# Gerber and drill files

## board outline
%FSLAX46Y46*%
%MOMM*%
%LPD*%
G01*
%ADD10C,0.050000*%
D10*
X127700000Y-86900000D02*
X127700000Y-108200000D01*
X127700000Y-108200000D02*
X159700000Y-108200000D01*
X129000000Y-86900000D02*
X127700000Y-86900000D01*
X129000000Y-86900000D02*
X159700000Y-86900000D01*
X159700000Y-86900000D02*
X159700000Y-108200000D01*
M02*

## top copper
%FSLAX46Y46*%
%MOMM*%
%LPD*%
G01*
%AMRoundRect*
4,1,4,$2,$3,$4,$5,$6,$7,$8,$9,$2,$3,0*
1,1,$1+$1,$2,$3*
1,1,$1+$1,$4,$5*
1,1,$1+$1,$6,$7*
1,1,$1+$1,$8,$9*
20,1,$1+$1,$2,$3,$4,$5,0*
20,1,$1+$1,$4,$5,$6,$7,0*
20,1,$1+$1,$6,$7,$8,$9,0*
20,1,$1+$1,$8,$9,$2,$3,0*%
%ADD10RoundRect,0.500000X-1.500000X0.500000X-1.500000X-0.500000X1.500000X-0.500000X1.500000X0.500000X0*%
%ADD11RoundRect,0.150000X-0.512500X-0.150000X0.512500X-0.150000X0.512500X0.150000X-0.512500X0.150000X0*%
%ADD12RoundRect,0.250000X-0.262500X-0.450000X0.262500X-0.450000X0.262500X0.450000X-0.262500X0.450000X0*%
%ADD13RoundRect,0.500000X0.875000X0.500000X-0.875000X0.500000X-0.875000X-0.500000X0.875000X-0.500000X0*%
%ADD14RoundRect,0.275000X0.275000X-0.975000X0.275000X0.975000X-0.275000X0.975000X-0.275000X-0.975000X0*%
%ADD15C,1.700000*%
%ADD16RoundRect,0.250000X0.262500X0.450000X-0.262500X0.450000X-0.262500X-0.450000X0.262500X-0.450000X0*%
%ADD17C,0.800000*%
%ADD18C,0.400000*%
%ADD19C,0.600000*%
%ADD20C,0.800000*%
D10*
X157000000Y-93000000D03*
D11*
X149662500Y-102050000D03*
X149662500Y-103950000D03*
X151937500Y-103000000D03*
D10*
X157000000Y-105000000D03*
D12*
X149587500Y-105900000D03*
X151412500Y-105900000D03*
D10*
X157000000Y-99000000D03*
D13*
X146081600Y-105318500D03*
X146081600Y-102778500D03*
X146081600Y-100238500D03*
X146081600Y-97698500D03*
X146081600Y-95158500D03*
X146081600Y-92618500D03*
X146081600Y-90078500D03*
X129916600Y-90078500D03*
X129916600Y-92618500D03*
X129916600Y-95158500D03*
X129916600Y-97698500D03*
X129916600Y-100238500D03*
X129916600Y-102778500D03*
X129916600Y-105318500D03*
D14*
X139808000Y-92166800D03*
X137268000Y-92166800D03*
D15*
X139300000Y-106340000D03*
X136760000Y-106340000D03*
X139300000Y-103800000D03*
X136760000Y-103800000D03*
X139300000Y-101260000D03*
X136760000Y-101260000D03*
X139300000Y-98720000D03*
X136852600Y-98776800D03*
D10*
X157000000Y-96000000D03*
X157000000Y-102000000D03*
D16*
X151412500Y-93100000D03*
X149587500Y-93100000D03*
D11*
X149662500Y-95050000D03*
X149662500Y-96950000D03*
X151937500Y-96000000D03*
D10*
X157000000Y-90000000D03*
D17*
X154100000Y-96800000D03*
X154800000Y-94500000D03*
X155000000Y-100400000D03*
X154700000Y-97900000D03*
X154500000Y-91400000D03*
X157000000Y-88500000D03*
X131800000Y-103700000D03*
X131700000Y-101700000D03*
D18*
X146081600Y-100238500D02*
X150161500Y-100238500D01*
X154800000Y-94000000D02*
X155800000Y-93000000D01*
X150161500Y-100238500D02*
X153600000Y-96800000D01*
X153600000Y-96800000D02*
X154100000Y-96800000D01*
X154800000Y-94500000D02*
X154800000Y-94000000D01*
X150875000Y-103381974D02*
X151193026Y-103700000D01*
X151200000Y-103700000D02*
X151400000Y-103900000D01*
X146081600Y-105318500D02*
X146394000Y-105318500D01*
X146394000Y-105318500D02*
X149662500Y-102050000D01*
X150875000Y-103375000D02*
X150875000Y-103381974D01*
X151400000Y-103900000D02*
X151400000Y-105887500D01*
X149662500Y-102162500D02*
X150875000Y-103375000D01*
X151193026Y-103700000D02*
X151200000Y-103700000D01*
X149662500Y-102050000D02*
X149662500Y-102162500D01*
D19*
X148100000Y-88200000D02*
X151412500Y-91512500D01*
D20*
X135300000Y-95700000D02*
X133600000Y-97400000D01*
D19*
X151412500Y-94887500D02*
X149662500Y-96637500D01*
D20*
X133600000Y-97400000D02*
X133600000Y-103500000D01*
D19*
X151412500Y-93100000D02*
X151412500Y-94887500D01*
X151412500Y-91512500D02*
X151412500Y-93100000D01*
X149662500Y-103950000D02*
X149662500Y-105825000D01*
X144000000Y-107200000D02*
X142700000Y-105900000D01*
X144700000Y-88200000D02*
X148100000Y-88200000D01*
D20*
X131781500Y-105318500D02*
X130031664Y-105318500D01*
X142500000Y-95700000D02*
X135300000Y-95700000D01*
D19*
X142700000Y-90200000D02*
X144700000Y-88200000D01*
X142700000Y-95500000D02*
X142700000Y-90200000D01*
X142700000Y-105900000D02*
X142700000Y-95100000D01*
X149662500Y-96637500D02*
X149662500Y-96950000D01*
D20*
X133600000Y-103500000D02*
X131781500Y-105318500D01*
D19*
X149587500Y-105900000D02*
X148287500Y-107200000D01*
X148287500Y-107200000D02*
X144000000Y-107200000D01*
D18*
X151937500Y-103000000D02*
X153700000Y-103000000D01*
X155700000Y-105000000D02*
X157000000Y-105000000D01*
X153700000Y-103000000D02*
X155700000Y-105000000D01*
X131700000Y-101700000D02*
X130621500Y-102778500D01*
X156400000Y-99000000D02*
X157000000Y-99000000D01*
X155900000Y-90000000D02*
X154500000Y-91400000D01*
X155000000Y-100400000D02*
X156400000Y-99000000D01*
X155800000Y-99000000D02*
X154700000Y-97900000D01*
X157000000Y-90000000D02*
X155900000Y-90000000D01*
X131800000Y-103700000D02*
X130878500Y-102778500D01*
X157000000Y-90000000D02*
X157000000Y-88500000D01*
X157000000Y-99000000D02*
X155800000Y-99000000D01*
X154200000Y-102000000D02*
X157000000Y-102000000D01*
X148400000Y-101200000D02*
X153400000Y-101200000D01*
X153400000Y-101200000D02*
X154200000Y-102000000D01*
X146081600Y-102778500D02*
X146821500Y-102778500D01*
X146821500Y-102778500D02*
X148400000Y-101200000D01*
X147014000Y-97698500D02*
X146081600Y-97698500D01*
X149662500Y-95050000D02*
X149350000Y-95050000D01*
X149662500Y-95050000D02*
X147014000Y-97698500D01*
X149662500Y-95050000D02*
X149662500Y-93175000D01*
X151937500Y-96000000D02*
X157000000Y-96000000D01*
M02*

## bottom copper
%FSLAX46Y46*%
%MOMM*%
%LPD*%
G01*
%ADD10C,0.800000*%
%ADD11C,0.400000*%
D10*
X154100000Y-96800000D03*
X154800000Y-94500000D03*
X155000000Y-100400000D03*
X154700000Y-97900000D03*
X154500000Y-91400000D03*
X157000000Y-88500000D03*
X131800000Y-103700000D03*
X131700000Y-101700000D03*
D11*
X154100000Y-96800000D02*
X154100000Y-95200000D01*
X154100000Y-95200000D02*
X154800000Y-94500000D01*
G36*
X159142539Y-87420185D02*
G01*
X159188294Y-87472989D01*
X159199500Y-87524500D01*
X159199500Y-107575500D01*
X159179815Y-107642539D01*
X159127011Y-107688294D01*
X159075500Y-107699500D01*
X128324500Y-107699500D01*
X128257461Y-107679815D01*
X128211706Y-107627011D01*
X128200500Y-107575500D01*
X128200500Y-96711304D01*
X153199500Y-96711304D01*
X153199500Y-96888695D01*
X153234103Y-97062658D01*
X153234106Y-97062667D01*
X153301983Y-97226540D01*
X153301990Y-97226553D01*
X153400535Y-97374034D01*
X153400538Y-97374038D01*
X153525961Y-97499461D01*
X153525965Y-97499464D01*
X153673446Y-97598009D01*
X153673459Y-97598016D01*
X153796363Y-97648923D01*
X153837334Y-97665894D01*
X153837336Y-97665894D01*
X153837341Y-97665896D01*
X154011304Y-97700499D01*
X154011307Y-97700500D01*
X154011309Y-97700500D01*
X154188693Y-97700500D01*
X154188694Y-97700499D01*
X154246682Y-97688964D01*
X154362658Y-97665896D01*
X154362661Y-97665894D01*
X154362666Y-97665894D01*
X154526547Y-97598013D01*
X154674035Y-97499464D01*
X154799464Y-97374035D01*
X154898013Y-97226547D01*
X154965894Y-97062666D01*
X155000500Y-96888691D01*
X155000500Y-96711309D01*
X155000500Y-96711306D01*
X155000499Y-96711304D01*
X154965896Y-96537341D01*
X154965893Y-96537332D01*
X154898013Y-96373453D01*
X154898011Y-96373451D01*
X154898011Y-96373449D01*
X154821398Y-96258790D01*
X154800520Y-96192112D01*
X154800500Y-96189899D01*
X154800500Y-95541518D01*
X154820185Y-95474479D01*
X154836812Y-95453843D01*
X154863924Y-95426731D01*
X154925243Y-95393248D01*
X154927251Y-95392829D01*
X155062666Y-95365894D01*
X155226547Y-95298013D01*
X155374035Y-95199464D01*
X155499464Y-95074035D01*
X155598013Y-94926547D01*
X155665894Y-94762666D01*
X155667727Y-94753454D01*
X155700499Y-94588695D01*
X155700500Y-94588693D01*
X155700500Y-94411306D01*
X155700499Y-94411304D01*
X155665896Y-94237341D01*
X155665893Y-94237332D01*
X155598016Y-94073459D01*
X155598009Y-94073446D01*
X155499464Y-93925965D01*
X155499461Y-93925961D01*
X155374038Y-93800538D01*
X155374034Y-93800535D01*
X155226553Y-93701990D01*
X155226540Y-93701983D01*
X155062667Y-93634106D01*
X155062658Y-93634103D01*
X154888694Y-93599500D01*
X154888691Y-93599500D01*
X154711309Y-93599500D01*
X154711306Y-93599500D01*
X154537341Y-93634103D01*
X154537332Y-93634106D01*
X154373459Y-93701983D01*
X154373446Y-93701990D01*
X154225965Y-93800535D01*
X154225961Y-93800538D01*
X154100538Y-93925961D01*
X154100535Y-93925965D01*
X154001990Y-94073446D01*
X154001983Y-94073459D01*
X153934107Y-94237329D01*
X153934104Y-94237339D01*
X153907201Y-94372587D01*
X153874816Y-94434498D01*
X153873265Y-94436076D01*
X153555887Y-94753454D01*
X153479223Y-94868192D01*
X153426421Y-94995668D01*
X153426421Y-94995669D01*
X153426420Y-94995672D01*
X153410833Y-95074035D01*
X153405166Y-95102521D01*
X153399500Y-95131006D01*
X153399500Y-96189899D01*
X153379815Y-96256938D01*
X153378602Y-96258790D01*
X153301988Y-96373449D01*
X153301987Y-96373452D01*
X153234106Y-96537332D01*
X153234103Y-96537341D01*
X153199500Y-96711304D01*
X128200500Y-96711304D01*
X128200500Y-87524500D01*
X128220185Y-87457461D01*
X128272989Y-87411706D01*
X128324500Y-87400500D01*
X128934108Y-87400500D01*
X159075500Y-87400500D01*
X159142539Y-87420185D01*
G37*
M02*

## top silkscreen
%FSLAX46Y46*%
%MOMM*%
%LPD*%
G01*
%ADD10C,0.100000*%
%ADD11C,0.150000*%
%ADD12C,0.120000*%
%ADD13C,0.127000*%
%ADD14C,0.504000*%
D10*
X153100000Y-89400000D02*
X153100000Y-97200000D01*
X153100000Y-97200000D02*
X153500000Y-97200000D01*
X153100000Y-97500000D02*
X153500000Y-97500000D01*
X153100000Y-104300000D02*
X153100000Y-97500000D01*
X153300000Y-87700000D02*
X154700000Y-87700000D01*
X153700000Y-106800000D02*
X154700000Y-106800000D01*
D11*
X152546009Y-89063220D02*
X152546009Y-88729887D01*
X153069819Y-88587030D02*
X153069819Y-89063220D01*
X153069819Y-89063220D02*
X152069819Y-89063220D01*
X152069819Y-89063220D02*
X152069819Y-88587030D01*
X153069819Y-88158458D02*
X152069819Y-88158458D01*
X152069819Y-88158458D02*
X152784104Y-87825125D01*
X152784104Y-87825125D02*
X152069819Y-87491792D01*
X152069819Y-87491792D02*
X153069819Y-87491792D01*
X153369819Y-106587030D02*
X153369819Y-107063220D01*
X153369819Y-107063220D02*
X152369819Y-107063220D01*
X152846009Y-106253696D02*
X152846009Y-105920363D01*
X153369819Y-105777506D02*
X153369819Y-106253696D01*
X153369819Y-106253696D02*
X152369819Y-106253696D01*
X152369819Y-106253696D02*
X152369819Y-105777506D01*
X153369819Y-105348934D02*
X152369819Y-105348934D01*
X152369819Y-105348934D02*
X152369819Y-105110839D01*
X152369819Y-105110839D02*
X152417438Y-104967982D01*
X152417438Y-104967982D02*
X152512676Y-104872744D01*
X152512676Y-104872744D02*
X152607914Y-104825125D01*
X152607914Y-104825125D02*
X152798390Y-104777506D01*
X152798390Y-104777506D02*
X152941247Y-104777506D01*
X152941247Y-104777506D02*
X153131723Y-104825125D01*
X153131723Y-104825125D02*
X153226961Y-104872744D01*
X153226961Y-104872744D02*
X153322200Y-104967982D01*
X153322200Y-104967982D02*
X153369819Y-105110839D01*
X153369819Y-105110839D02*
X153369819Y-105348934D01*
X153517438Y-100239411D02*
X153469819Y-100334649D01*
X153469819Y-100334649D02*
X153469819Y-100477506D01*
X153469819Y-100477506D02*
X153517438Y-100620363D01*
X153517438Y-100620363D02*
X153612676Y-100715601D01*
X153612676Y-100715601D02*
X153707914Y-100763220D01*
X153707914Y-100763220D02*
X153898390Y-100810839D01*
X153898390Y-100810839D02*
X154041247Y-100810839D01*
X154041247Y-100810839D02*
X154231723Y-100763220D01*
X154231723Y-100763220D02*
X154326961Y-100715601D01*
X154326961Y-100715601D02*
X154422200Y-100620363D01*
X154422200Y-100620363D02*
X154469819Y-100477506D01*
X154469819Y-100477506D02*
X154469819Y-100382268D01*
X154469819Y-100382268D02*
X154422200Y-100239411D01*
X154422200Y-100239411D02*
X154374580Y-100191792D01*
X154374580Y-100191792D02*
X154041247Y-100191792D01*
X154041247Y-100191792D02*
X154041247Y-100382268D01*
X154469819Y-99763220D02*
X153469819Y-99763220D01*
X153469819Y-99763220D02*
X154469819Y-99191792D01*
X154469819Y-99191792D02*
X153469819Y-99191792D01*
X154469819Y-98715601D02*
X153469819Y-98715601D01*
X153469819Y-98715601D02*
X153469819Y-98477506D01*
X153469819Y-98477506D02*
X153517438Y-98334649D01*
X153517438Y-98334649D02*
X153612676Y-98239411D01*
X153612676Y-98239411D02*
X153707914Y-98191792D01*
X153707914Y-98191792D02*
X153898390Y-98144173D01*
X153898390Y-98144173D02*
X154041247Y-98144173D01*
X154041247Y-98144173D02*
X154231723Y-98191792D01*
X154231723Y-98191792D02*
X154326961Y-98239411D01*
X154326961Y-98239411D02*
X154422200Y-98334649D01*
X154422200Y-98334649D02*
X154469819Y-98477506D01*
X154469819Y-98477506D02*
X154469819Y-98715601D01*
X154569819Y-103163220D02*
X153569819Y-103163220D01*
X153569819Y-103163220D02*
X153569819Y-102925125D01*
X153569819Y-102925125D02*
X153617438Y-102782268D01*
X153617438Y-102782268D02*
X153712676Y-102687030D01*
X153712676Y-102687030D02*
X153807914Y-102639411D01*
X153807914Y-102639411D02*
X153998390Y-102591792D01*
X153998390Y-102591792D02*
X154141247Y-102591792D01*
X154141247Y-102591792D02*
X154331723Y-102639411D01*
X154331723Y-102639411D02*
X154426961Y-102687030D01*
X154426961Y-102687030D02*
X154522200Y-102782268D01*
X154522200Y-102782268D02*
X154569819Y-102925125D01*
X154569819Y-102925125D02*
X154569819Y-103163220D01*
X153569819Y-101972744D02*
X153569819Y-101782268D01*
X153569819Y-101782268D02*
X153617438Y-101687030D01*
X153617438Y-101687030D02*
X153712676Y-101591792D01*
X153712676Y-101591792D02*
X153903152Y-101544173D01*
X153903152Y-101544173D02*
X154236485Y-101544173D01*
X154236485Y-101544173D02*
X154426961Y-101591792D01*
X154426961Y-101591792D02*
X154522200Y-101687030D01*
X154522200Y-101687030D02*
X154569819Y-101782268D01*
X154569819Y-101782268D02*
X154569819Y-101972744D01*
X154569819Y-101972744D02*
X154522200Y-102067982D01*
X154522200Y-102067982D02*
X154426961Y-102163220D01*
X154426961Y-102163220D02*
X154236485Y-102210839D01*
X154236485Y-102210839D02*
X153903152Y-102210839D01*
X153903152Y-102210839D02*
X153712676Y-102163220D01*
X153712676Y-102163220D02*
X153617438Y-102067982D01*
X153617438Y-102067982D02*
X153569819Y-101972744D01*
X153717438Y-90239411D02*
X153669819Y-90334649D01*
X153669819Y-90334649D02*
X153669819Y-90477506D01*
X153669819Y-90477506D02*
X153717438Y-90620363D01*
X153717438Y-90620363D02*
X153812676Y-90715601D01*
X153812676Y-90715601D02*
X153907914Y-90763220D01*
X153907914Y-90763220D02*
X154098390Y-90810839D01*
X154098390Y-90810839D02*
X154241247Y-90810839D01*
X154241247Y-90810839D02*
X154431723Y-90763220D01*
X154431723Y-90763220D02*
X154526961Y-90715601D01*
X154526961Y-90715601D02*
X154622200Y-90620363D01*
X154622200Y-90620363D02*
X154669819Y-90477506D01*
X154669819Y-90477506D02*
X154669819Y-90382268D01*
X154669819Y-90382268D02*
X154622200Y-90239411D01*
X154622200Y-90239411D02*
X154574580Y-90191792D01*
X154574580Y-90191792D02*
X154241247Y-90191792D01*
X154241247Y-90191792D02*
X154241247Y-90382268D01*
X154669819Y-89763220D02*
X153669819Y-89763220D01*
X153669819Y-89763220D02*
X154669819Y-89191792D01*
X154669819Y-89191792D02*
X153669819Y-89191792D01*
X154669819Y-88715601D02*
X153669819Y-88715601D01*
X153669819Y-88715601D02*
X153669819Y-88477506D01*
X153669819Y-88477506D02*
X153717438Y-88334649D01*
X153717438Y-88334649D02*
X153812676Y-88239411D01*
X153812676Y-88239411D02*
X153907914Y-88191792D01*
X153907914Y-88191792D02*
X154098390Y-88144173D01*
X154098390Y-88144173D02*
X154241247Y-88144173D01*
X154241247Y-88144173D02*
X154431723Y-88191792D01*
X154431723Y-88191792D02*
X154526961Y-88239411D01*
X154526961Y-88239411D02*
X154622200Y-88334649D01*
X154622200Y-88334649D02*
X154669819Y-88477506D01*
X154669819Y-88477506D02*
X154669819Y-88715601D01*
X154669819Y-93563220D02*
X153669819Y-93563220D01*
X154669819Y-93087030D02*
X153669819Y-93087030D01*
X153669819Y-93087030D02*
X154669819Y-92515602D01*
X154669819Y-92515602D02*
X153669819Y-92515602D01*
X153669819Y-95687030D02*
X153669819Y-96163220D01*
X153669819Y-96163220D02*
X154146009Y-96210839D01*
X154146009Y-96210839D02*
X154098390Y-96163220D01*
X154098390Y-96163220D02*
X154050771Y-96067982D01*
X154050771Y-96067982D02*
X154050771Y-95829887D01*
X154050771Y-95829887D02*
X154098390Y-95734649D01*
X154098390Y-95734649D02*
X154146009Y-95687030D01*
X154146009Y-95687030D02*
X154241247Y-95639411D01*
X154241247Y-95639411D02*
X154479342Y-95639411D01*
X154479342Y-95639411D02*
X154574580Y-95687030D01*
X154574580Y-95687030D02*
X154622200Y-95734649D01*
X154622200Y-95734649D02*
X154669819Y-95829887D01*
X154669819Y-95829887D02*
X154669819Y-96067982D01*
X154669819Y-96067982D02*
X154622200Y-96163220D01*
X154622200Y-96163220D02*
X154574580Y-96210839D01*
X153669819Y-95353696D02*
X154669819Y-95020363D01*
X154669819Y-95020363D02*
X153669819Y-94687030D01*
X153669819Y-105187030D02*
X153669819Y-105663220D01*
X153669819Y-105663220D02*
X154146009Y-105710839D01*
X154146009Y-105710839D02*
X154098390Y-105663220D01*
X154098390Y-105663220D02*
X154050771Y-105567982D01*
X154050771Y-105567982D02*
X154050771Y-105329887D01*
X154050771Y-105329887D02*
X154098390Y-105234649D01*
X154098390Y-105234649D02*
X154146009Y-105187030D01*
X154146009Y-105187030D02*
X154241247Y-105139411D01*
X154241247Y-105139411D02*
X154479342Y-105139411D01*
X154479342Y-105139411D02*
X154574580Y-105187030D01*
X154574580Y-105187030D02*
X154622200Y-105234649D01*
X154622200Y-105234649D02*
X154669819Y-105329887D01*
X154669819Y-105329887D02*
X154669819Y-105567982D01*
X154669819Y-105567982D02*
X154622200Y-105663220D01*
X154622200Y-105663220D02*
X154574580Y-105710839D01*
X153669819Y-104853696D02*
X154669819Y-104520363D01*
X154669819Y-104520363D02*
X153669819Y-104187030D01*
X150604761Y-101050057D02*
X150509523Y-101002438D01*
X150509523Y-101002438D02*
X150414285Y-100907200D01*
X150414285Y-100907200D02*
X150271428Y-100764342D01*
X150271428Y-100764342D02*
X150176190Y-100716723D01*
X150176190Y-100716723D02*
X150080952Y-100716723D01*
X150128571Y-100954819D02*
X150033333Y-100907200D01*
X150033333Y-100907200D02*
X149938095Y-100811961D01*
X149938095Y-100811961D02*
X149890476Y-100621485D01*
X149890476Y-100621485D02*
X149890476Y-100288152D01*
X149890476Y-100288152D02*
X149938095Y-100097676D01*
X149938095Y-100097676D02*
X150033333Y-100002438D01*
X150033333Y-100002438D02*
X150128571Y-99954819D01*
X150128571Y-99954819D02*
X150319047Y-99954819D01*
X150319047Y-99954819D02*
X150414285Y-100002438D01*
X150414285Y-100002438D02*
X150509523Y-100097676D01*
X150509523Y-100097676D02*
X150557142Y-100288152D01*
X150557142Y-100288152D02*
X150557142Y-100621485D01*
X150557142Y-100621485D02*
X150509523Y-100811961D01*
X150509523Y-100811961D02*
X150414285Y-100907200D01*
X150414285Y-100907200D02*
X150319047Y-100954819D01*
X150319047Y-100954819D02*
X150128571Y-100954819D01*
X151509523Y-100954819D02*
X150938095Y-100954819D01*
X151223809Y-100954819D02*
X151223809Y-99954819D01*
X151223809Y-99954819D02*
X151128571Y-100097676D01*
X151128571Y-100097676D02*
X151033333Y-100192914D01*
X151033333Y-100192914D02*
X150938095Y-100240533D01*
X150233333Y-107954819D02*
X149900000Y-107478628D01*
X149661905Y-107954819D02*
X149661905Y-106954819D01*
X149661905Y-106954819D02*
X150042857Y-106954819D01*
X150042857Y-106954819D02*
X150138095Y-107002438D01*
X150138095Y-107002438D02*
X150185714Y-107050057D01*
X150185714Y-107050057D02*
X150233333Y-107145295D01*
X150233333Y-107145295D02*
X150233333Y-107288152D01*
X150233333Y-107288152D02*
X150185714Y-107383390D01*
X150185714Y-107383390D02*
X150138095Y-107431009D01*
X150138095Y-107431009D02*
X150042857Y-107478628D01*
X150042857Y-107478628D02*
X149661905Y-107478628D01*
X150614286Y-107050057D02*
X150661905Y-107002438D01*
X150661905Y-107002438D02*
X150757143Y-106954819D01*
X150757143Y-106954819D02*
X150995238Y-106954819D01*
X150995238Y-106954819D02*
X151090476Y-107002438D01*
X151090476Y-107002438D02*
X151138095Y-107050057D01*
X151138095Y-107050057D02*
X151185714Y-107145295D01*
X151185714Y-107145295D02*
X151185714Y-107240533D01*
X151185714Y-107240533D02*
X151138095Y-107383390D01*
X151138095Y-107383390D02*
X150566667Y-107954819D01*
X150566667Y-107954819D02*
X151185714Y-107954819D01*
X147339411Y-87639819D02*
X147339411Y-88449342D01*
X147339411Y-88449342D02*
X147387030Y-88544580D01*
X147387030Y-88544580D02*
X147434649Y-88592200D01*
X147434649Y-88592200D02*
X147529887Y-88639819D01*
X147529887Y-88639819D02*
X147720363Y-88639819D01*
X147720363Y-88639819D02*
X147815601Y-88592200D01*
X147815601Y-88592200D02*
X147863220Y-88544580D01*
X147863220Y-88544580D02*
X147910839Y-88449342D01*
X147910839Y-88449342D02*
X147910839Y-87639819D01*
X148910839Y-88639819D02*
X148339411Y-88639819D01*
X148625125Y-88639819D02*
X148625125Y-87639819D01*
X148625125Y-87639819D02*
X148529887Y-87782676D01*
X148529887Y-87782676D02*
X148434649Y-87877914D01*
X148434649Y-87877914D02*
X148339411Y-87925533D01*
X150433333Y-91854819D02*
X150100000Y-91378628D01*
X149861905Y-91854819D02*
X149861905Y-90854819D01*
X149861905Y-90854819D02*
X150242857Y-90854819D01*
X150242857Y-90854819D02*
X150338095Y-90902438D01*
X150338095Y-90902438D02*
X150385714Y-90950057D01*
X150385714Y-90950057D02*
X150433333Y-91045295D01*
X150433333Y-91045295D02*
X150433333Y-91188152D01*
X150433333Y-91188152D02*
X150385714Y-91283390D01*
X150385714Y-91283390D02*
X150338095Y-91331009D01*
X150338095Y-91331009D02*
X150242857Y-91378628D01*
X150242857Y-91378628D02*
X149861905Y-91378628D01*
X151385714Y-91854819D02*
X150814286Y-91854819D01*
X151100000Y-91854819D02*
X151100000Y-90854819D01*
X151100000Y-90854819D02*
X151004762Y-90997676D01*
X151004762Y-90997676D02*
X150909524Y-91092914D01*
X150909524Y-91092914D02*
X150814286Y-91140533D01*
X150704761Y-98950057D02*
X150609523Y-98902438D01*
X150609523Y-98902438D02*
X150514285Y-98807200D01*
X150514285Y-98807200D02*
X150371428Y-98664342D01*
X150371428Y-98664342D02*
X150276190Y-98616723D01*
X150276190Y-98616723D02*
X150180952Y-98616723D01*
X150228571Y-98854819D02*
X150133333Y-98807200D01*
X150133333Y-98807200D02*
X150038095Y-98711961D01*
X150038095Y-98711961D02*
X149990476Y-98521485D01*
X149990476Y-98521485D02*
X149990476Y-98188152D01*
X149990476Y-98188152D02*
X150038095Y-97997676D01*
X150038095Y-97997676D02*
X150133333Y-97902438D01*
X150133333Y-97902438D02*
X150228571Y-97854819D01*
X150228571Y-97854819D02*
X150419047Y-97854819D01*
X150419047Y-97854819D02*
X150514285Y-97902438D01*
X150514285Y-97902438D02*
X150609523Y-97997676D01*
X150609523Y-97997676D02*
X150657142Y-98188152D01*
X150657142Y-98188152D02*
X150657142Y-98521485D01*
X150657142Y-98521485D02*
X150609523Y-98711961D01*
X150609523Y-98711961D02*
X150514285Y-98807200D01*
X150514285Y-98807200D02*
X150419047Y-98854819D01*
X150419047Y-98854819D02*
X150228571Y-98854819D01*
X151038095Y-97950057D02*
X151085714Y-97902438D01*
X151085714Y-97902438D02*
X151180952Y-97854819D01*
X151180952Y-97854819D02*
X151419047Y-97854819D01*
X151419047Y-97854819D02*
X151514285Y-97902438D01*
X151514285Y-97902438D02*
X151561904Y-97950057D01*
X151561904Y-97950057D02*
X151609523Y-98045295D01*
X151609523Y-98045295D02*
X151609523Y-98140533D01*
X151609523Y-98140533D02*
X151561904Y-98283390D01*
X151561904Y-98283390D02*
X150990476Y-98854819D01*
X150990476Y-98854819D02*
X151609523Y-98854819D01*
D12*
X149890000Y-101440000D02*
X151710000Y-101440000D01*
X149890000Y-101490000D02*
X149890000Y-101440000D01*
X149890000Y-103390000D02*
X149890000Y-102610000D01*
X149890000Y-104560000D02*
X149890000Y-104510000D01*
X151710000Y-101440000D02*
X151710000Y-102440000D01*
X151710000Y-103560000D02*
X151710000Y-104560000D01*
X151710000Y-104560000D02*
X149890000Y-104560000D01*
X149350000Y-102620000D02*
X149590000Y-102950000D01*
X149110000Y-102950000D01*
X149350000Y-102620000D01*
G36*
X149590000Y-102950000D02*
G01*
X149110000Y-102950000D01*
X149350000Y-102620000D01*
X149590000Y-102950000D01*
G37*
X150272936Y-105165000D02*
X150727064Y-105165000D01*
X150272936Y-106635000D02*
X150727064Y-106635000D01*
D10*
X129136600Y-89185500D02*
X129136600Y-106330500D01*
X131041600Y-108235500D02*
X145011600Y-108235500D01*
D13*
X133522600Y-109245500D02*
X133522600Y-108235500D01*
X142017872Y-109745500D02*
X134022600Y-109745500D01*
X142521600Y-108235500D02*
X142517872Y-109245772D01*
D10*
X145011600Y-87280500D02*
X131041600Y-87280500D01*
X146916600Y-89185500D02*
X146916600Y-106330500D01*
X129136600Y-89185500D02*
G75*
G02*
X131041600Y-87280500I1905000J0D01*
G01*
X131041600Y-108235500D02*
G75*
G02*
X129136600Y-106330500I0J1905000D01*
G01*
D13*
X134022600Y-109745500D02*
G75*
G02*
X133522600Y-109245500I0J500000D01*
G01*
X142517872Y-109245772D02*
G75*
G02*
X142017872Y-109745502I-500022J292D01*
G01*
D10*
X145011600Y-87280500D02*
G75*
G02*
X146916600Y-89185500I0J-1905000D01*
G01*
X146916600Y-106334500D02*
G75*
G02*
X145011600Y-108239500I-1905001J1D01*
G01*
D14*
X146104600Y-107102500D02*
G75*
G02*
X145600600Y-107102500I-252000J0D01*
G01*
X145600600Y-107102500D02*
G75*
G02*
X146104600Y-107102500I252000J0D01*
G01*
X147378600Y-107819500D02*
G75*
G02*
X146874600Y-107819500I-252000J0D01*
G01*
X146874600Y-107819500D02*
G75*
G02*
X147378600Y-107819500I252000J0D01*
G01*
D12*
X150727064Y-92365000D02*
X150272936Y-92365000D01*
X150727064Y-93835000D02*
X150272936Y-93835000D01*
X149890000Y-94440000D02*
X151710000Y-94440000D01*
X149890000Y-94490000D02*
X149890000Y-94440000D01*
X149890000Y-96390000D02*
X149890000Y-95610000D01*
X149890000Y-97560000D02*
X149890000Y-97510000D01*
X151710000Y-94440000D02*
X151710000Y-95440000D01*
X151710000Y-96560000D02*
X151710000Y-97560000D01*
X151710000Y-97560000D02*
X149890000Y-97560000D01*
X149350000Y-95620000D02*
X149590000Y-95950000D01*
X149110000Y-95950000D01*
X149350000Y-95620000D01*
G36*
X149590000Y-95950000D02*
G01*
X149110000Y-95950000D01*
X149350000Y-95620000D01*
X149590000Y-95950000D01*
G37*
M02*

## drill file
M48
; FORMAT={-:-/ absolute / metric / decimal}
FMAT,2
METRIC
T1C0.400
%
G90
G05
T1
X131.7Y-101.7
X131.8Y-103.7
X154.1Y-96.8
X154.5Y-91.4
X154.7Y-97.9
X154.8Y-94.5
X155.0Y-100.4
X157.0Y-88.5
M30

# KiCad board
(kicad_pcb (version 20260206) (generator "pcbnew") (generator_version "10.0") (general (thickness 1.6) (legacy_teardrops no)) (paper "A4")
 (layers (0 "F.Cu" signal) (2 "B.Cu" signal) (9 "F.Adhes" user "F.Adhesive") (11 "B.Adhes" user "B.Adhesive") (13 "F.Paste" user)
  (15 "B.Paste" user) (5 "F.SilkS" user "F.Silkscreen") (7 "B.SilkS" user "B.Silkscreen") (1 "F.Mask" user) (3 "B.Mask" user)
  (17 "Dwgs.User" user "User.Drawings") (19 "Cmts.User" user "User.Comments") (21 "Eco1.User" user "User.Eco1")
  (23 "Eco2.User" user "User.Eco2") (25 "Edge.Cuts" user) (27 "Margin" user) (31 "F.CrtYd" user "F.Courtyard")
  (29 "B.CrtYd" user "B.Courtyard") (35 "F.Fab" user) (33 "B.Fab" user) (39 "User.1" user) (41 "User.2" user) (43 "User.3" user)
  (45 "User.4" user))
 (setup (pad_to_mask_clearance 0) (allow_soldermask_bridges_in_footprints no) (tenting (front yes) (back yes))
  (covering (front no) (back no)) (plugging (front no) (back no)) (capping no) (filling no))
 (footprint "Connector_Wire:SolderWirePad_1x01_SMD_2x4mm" (layer "F.Cu") (at 157 93 -90)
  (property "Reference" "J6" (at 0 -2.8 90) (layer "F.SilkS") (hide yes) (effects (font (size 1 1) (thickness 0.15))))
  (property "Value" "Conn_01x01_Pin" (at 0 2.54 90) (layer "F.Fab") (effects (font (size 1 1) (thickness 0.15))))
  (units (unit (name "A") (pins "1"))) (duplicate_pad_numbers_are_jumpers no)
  (pad "1" smd roundrect (at 0 0 270) (size 2 4) (layers "F.Cu" "F.Mask") (roundrect_rratio 0.25) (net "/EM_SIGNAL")))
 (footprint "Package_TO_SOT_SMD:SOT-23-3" (layer "F.Cu") (at 150.8 103)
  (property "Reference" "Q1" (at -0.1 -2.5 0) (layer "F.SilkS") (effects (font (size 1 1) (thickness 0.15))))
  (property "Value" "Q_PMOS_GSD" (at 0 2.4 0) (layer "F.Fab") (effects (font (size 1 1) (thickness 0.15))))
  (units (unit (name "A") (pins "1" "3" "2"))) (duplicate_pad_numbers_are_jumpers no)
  (fp_line (start -0.91 -1.56) (end 0.91 -1.56) (stroke (width 0.12) (type solid)) (layer "F.SilkS"))
  (fp_line (start -0.91 -1.51) (end -0.91 -1.56) (stroke (width 0.12) (type solid)) (layer "F.SilkS"))
  (fp_line (start -0.91 0.39) (end -0.91 -0.39) (stroke (width 0.12) (type solid)) (layer "F.SilkS"))
  (fp_line (start -0.91 1.56) (end -0.91 1.51) (stroke (width 0.12) (type solid)) (layer "F.SilkS"))
  (fp_line (start 0.91 -1.56) (end 0.91 -0.56) (stroke (width 0.12) (type solid)) (layer "F.SilkS"))
  (fp_line (start 0.91 0.56) (end 0.91 1.56) (stroke (width 0.12) (type solid)) (layer "F.SilkS"))
  (fp_line (start 0.91 1.56) (end -0.91 1.56) (stroke (width 0.12) (type solid)) (layer "F.SilkS"))
  (fp_poly (pts (xy -1.45 -0.38) (xy -1.21 -0.05) (xy -1.69 -0.05)) (stroke (width 0.12) (type solid)) (fill yes) (layer "F.SilkS"))
  (pad "1" smd roundrect (at -1.1375 -0.95) (size 1.325 0.6) (layers "F.Cu" "F.Mask" "F.Paste") (roundrect_rratio 0.25) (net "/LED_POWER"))
  (pad "2" smd roundrect (at -1.1375 0.95) (size 1.325 0.6) (layers "F.Cu" "F.Mask" "F.Paste") (roundrect_rratio 0.25) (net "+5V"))
  (pad "3" smd roundrect (at 1.1375 0) (size 1.325 0.6) (layers "F.Cu" "F.Mask" "F.Paste") (roundrect_rratio 0.25) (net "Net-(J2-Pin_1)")))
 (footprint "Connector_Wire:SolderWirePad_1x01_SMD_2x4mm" (layer "F.Cu") (at 157 105 -90)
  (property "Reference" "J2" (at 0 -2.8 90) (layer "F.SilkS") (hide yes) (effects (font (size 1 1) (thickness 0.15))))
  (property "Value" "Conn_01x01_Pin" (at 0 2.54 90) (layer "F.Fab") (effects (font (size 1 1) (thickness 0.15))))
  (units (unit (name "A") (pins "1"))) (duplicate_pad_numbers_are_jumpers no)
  (pad "1" smd roundrect (at 0 0 270) (size 2 4) (layers "F.Cu" "F.Mask") (roundrect_rratio 0.25) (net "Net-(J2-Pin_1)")))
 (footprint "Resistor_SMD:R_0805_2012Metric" (layer "F.Cu") (at 150.5 105.9)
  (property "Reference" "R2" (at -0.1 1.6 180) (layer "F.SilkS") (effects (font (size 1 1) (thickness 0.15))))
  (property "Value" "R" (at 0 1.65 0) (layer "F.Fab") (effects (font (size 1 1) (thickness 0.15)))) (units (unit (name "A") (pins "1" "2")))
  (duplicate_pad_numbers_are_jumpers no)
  (fp_line (start -0.227064 -0.735) (end 0.227064 -0.735) (stroke (width 0.12) (type solid)) (layer "F.SilkS"))
  (fp_line (start -0.227064 0.735) (end 0.227064 0.735) (stroke (width 0.12) (type solid)) (layer "F.SilkS"))
  (pad "1" smd roundrect (at -0.9125 0) (size 1.025 1.4) (layers "F.Cu" "F.Mask" "F.Paste") (roundrect_rratio 0.243902) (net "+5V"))
  (pad "2" smd roundrect (at 0.9125 0) (size 1.025 1.4) (layers "F.Cu" "F.Mask" "F.Paste") (roundrect_rratio 0.243902) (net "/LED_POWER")))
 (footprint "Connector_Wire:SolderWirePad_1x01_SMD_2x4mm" (layer "F.Cu") (at 157 99 -90)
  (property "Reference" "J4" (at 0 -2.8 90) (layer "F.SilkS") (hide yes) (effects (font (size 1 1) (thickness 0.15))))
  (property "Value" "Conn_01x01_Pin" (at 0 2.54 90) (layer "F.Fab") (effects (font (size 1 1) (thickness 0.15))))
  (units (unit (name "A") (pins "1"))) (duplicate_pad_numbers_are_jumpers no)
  (pad "1" smd roundrect (at 0 0 270) (size 2 4) (layers "F.Cu" "F.Mask") (roundrect_rratio 0.25) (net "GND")))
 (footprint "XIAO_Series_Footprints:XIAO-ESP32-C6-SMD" (layer "F.Cu") (at 146.9166 87.1985 180)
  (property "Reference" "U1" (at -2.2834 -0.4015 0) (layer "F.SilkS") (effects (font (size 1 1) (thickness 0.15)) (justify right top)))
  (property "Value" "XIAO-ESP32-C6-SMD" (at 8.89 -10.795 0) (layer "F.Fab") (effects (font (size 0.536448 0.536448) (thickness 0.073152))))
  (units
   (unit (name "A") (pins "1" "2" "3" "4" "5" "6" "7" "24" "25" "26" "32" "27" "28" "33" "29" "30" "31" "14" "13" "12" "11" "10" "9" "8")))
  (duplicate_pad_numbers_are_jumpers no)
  (fp_line (start 17.78 -1.987) (end 17.78 -19.132) (stroke (width 0.1) (type solid)) (layer "F.SilkS"))
  (fp_line (start 15.875 -21.037) (end 1.905 -21.037) (stroke (width 0.1) (type solid)) (layer "F.SilkS"))
  (fp_line (start 13.394 -22.047) (end 13.394 -21.037) (stroke (width 0.127) (type solid)) (layer "F.SilkS"))
  (fp_line (start 4.898728 -22.547) (end 12.894 -22.547) (stroke (width 0.127) (type solid)) (layer "F.SilkS"))
  (fp_line (start 4.395 -21.037) (end 4.398728 -22.047272) (stroke (width 0.127) (type solid)) (layer "F.SilkS"))
  (fp_line (start 1.905 -0.082) (end 15.875 -0.082) (stroke (width 0.1) (type solid)) (layer "F.SilkS"))
  (fp_line (start 0 -1.987) (end 0 -19.132) (stroke (width 0.1) (type solid)) (layer "F.SilkS"))
  (fp_arc (start 17.78 -1.987) (mid 17.222038 -0.639962) (end 15.875 -0.082) (stroke (width 0.1) (type solid)) (layer "F.SilkS"))
  (fp_arc (start 15.875 -21.037) (mid 17.222038 -20.479038) (end 17.78 -19.132) (stroke (width 0.1) (type solid)) (layer "F.SilkS"))
  (fp_arc (start 12.894 -22.547) (mid 13.247553 -22.400553) (end 13.394 -22.047) (stroke (width 0.127) (type default)) (layer "F.SilkS"))
  (fp_arc (start 4.398728 -22.047272) (mid 4.545276 -22.400644) (end 4.898728 -22.547) (stroke (width 0.127) (type default))
   (layer "F.SilkS"))
  (fp_arc (start 1.905 -0.082) (mid 0.557962 -0.639962) (end 0 -1.987) (stroke (width 0.1) (type solid)) (layer "F.SilkS"))
  (fp_arc (start 0 -19.136) (mid 0.557962 -20.483038) (end 1.905 -21.041) (stroke (width 0.1) (type solid)) (layer "F.SilkS"))
  (fp_circle (center 1.064 -19.904) (end 1.064 -20.158) (stroke (width 0.5) (type solid)) (fill yes) (layer "F.SilkS"))
  (fp_circle (center -0.21 -20.621) (end -0.21 -20.875) (stroke (width 0.5) (type solid)) (fill yes) (layer "F.SilkS"))
  (pad "1" smd roundrect (at 0.835 -18.12 180) (size 2.75 2) (layers "F.Cu" "F.Mask" "F.Paste") (roundrect_rratio 0.25) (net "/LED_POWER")
   (solder_mask_margin 0.0508) (thermal_bridge_angle 45))
  (pad "2" smd roundrect (at 0.835 -15.58 180) (size 2.75 2) (layers "F.Cu" "F.Mask" "F.Paste") (roundrect_rratio 0.25) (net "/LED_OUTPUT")
   (solder_mask_margin 0.0508) (thermal_bridge_angle 45))
  (pad "3" smd roundrect (at 0.835 -13.04 180) (size 2.75 2) (layers "F.Cu" "F.Mask" "F.Paste") (roundrect_rratio 0.25) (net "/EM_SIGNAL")
   (solder_mask_margin 0.0508) (thermal_bridge_angle 45))
  (pad "4" smd roundrect (at 0.835 -10.5 180) (size 2.75 2) (layers "F.Cu" "F.Mask" "F.Paste") (roundrect_rratio 0.25) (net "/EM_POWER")
   (solder_mask_margin 0.0508) (thermal_bridge_angle 45))
  (pad "5" smd roundrect (at 0.835 -7.96 180) (size 2.75 2) (layers "F.Cu" "F.Mask" "F.Paste") (roundrect_rratio 0.25)
   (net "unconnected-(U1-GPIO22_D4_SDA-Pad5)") (solder_mask_margin 0.0508) (thermal_bridge_angle 45))
  (pad "6" smd roundrect (at 0.835 -5.42 180) (size 2.75 2) (layers "F.Cu" "F.Mask" "F.Paste") (roundrect_rratio 0.25)
   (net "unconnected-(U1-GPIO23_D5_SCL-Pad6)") (solder_mask_margin 0.0508) (thermal_bridge_angle 45))
  (pad "7" smd roundrect (at 0.835 -2.88 180) (size 2.75 2) (layers "F.Cu" "F.Mask" "F.Paste") (roundrect_rratio 0.25)
   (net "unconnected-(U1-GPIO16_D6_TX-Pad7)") (solder_mask_margin 0.0508) (thermal_bridge_angle 45))
  (pad "8" smd roundrect (at 17 -2.88 180) (size 2.75 2) (layers "F.Cu" "F.Mask" "F.Paste") (roundrect_rratio 0.25)
   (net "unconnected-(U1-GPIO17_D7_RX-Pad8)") (solder_mask_margin 0.0508) (thermal_bridge_angle 45))
  (pad "9" smd roundrect (at 17 -5.42 180) (size 2.75 2) (layers "F.Cu" "F.Mask" "F.Paste") (roundrect_rratio 0.25)
   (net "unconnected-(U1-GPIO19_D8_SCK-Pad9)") (solder_mask_margin 0.0508) (thermal_bridge_angle 45))
  (pad "10" smd roundrect (at 17 -7.96 180) (size 2.75 2) (layers "F.Cu" "F.Mask" "F.Paste") (roundrect_rratio 0.25)
   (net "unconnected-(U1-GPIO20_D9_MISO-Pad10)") (solder_mask_margin 0.0508) (thermal_bridge_angle 45))
  (pad "11" smd roundrect (at 17 -10.5 180) (size 2.75 2) (layers "F.Cu" "F.Mask" "F.Paste") (roundrect_rratio 0.25)
   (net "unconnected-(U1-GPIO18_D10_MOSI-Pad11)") (solder_mask_margin 0.0508) (thermal_bridge_angle 45))
  (pad "12" smd roundrect (at 17 -13.04 180) (size 2.75 2) (layers "F.Cu" "F.Mask" "F.Paste") (roundrect_rratio 0.25)
   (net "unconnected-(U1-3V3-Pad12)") (solder_mask_margin 0.0508) (thermal_bridge_angle 45))
  (pad "13" smd roundrect (at 17 -15.58 180) (size 2.75 2) (layers "F.Cu" "F.Mask" "F.Paste") (roundrect_rratio 0.25) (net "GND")
   (solder_mask_margin 0.0508) (thermal_bridge_angle 45))
  (pad "14" smd roundrect (at 17 -18.12 180) (size 2.75 2) (layers "F.Cu" "F.Mask" "F.Paste") (roundrect_rratio 0.25) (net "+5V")
   (solder_mask_margin 0.0508) (thermal_bridge_angle 45))
  (pad "15" smd roundrect (at 7.1086 -4.9683 90) (size 2.5 1.1) (layers "F.Cu" "F.Mask" "F.Paste") (roundrect_rratio 0.25)
   (solder_mask_margin 0.0508) (thermal_bridge_angle 45))
  (pad "16" smd roundrect (at 9.6486 -4.9683 90) (size 2.5 1.1) (layers "F.Cu" "F.Mask" "F.Paste") (roundrect_rratio 0.25)
   (solder_mask_margin 0.0508) (thermal_bridge_angle 45))
  (pad "17" smd circle (at 7.6166 -19.1415 180) (size 1.7 1.7) (layers "F.Cu" "F.Mask" "F.Paste"))
  (pad "18" smd circle (at 10.1566 -19.1415 180) (size 1.7 1.7) (layers "F.Cu" "F.Mask" "F.Paste"))
  (pad "19" smd circle (at 7.6166 -16.6015 180) (size 1.7 1.7) (layers "F.Cu" "F.Mask" "F.Paste"))
  (pad "20" smd circle (at 10.1566 -16.6015 180) (size 1.7 1.7) (layers "F.Cu" "F.Mask" "F.Paste"))
  (pad "21" smd circle (at 7.6166 -14.0615 180) (size 1.7 1.7) (layers "F.Cu" "F.Mask" "F.Paste"))
  (pad "22" smd circle (at 10.1566 -14.0615 180) (size 1.7 1.7) (layers "F.Cu" "F.Mask" "F.Paste"))
  (pad "23" smd circle (at 7.6166 -11.5215 180) (size 1.7 1.7) (layers "F.Cu" "F.Mask" "F.Paste"))
  (pad "24" smd circle (at 10.064 -11.5783 180) (size 1.7 1.7) (layers "F.Cu" "F.Mask" "F.Paste") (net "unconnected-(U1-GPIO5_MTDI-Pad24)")))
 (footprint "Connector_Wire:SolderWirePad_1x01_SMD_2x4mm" (layer "F.Cu") (at 157 96 -90)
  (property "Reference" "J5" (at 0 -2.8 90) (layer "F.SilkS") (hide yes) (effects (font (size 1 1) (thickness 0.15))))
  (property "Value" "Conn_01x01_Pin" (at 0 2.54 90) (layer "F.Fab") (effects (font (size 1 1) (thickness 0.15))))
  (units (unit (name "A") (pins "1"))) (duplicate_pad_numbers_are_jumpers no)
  (pad "1" smd roundrect (at 0 0 270) (size 2 4) (layers "F.Cu" "F.Mask") (roundrect_rratio 0.25) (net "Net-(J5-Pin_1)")))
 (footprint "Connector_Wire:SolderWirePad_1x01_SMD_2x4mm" (layer "F.Cu") (at 157 102 -90)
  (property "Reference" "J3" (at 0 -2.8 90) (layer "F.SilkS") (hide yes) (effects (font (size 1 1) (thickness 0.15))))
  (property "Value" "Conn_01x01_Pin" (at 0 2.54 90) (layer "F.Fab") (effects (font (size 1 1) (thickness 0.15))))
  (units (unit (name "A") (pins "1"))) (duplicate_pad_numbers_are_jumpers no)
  (pad "1" smd roundrect (at 0 0 270) (size 2 4) (layers "F.Cu" "F.Mask") (roundrect_rratio 0.25) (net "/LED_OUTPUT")))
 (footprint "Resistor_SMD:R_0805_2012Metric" (layer "F.Cu") (at 150.5 93.1 180)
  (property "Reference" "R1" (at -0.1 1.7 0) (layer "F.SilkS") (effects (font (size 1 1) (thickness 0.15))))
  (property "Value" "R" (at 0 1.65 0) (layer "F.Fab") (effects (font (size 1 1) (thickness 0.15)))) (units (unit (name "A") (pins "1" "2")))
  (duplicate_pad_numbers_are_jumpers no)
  (fp_line (start -0.227064 0.735) (end 0.227064 0.735) (stroke (width 0.12) (type solid)) (layer "F.SilkS"))
  (fp_line (start -0.227064 -0.735) (end 0.227064 -0.735) (stroke (width 0.12) (type solid)) (layer "F.SilkS"))
  (pad "1" smd roundrect (at -0.9125 0 180) (size 1.025 1.4) (layers "F.Cu" "F.Mask" "F.Paste") (roundrect_rratio 0.243902) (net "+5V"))
  (pad "2" smd roundrect (at 0.9125 0 180) (size 1.025 1.4) (layers "F.Cu" "F.Mask" "F.Paste") (roundrect_rratio 0.243902) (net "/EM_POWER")))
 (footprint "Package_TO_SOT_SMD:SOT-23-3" (layer "F.Cu") (at 150.8 96)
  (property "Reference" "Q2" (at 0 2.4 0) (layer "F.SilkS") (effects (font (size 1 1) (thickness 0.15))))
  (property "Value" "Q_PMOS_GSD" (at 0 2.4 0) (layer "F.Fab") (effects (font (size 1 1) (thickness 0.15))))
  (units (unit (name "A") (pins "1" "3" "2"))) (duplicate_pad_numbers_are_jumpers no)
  (fp_line (start -0.91 -1.56) (end 0.91 -1.56) (stroke (width 0.12) (type solid)) (layer "F.SilkS"))
  (fp_line (start -0.91 -1.51) (end -0.91 -1.56) (stroke (width 0.12) (type solid)) (layer "F.SilkS"))
  (fp_line (start -0.91 0.39) (end -0.91 -0.39) (stroke (width 0.12) (type solid)) (layer "F.SilkS"))
  (fp_line (start -0.91 1.56) (end -0.91 1.51) (stroke (width 0.12) (type solid)) (layer "F.SilkS"))
  (fp_line (start 0.91 -1.56) (end 0.91 -0.56) (stroke (width 0.12) (type solid)) (layer "F.SilkS"))
  (fp_line (start 0.91 0.56) (end 0.91 1.56) (stroke (width 0.12) (type solid)) (layer "F.SilkS"))
  (fp_line (start 0.91 1.56) (end -0.91 1.56) (stroke (width 0.12) (type solid)) (layer "F.SilkS"))
  (fp_poly (pts (xy -1.45 -0.38) (xy -1.21 -0.05) (xy -1.69 -0.05)) (stroke (width 0.12) (type solid)) (fill yes) (layer "F.SilkS"))
  (pad "1" smd roundrect (at -1.1375 -0.95) (size 1.325 0.6) (layers "F.Cu" "F.Mask" "F.Paste") (roundrect_rratio 0.25) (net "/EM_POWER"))
  (pad "2" smd roundrect (at -1.1375 0.95) (size 1.325 0.6) (layers "F.Cu" "F.Mask" "F.Paste") (roundrect_rratio 0.25) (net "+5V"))
  (pad "3" smd roundrect (at 1.1375 0) (size 1.325 0.6) (layers "F.Cu" "F.Mask" "F.Paste") (roundrect_rratio 0.25) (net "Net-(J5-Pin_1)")))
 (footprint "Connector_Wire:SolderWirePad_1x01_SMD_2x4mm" (layer "F.Cu") (at 157 90 -90)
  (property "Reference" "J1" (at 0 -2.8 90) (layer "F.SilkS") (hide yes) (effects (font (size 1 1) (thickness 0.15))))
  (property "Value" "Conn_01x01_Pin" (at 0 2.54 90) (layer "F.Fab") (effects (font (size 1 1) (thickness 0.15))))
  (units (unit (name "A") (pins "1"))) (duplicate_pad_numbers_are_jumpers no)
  (pad "1" smd roundrect (at 0 0 270) (size 2 4) (layers "F.Cu" "F.Mask") (roundrect_rratio 0.25) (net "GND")))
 (gr_line (start 153.1 89.4) (end 153.1 97.2) (stroke (width 0.1) (type default)) (layer "F.SilkS"))
 (gr_line (start 153.1 97.2) (end 153.5 97.2) (stroke (width 0.1) (type default)) (layer "F.SilkS"))
 (gr_line (start 153.1 97.5) (end 153.5 97.5) (stroke (width 0.1) (type default)) (layer "F.SilkS"))
 (gr_line (start 153.1 104.3) (end 153.1 97.5) (stroke (width 0.1) (type default)) (layer "F.SilkS"))
 (gr_line (start 153.3 87.7) (end 154.7 87.7) (stroke (width 0.1) (type default)) (layer "F.SilkS"))
 (gr_line (start 153.7 106.8) (end 154.7 106.8) (stroke (width 0.1) (type default)) (layer "F.SilkS"))
 (gr_line (start 127.7 86.9) (end 127.7 108.2) (stroke (width 0.05) (type default)) (layer "Edge.Cuts"))
 (gr_line (start 127.7 108.2) (end 159.7 108.2) (stroke (width 0.05) (type default)) (layer "Edge.Cuts"))
 (gr_line (start 129 86.9) (end 127.7 86.9) (stroke (width 0.05) (type default)) (layer "Edge.Cuts"))
 (gr_line (start 129 86.9) (end 159.7 86.9) (stroke (width 0.05) (type default)) (layer "Edge.Cuts"))
 (gr_line (start 159.7 86.9) (end 159.7 108.2) (stroke (width 0.05) (type default)) (layer "Edge.Cuts"))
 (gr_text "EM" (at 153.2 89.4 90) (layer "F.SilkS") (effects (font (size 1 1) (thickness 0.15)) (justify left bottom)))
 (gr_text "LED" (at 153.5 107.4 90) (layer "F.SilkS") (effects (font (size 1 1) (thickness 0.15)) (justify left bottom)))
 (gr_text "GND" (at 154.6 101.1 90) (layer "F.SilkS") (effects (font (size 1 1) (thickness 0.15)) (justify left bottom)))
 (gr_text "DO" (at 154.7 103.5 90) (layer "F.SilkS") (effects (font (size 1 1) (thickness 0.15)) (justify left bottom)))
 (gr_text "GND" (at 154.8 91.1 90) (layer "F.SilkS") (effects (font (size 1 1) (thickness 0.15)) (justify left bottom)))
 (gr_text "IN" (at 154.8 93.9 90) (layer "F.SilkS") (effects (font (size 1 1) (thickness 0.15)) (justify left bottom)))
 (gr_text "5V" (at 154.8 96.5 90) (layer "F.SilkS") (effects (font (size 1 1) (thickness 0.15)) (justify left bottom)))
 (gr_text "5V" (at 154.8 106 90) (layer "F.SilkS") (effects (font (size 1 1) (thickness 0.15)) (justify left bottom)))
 (segment (start 146.0816 100.2385) (end 150.1615 100.2385) (width 0.4) (layer "F.Cu") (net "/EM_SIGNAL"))
 (segment (start 154.8 94) (end 155.8 93) (width 0.4) (layer "F.Cu") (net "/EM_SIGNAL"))
 (segment (start 150.1615 100.2385) (end 153.6 96.8) (width 0.4) (layer "F.Cu") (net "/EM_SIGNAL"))
 (segment (start 153.6 96.8) (end 154.1 96.8) (width 0.4) (layer "F.Cu") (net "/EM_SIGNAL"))
 (segment (start 154.8 94.5) (end 154.8 94) (width 0.4) (layer "F.Cu") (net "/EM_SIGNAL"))
 (via (at 154.1 96.8) (size 0.8) (drill 0.4) (layers "F.Cu" "B.Cu") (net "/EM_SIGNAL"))
 (via (at 154.8 94.5) (size 0.8) (drill 0.4) (layers "F.Cu" "B.Cu") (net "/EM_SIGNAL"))
 (segment (start 154.1 96.8) (end 154.1 95.2) (width 0.4) (layer "B.Cu") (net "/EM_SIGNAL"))
 (segment (start 154.1 95.2) (end 154.8 94.5) (width 0.4) (layer "B.Cu") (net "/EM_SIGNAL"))
 (segment (start 150.875 103.381974) (end 151.193026 103.7) (width 0.4) (layer "F.Cu") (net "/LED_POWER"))
 (segment (start 151.2 103.7) (end 151.4 103.9) (width 0.4) (layer "F.Cu") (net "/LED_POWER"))
 (segment (start 146.0816 105.3185) (end 146.394 105.3185) (width 0.4) (layer "F.Cu") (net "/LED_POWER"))
 (segment (start 146.394 105.3185) (end 149.6625 102.05) (width 0.4) (layer "F.Cu") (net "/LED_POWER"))
 (segment (start 150.875 103.375) (end 150.875 103.381974) (width 0.4) (layer "F.Cu") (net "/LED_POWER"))
 (segment (start 151.4 103.9) (end 151.4 105.8875) (width 0.4) (layer "F.Cu") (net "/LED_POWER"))
 (segment (start 149.6625 102.1625) (end 150.875 103.375) (width 0.4) (layer "F.Cu") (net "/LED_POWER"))
 (segment (start 151.193026 103.7) (end 151.2 103.7) (width 0.4) (layer "F.Cu") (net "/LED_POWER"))
 (segment (start 149.6625 102.05) (end 149.6625 102.1625) (width 0.4) (layer "F.Cu") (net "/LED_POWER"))
 (segment (start 148.1 88.2) (end 151.4125 91.5125) (width 0.6) (layer "F.Cu") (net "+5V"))
 (segment (start 135.3 95.7) (end 133.6 97.4) (width 0.8) (layer "F.Cu") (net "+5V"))
 (segment (start 151.4125 94.8875) (end 149.6625 96.6375) (width 0.6) (layer "F.Cu") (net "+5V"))
 (segment (start 133.6 97.4) (end 133.6 103.5) (width 0.8) (layer "F.Cu") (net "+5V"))
 (segment (start 151.4125 93.1) (end 151.4125 94.8875) (width 0.6) (layer "F.Cu") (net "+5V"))
 (segment (start 151.4125 91.5125) (end 151.4125 93.1) (width 0.6) (layer "F.Cu") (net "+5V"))
 (segment (start 149.6625 103.95) (end 149.6625 105.825) (width 0.6) (layer "F.Cu") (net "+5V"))
 (segment (start 144 107.2) (end 142.7 105.9) (width 0.6) (layer "F.Cu") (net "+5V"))
 (segment (start 144.7 88.2) (end 148.1 88.2) (width 0.6) (layer "F.Cu") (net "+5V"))
 (segment (start 131.7815 105.3185) (end 130.031664 105.3185) (width 0.8) (layer "F.Cu") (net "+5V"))
 (segment (start 142.5 95.7) (end 135.3 95.7) (width 0.8) (layer "F.Cu") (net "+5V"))
 (segment (start 142.7 90.2) (end 144.7 88.2) (width 0.6) (layer "F.Cu") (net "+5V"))
 (segment (start 142.7 95.5) (end 142.7 90.2) (width 0.6) (layer "F.Cu") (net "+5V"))
 (segment (start 142.7 105.9) (end 142.7 95.1) (width 0.6) (layer "F.Cu") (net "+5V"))
 (segment (start 149.6625 96.6375) (end 149.6625 96.95) (width 0.6) (layer "F.Cu") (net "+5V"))
 (segment (start 133.6 103.5) (end 131.7815 105.3185) (width 0.8) (layer "F.Cu") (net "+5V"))
 (segment (start 149.5875 105.9) (end 148.2875 107.2) (width 0.6) (layer "F.Cu") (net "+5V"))
 (segment (start 148.2875 107.2) (end 144 107.2) (width 0.6) (layer "F.Cu") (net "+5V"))
 (segment (start 151.9375 103) (end 153.7 103) (width 0.4) (layer "F.Cu") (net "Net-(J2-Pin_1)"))
 (segment (start 155.7 105) (end 157 105) (width 0.4) (layer "F.Cu") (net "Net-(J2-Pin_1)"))
 (segment (start 153.7 103) (end 155.7 105) (width 0.4) (layer "F.Cu") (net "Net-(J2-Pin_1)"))
 (segment (start 131.7 101.7) (end 130.6215 102.7785) (width 0.4) (layer "F.Cu") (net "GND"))
 (segment (start 156.4 99) (end 157 99) (width 0.4) (layer "F.Cu") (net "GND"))
 (segment (start 155.9 90) (end 154.5 91.4) (width 0.4) (layer "F.Cu") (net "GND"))
 (segment (start 155 100.4) (end 156.4 99) (width 0.4) (layer "F.Cu") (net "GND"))
 (segment (start 155.8 99) (end 154.7 97.9) (width 0.4) (layer "F.Cu") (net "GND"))
 (segment (start 157 90) (end 155.9 90) (width 0.4) (layer "F.Cu") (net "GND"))
 (segment (start 131.8 103.7) (end 130.8785 102.7785) (width 0.4) (layer "F.Cu") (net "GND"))
 (segment (start 157 90) (end 157 88.5) (width 0.4) (layer "F.Cu") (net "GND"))
 (segment (start 157 99) (end 155.8 99) (width 0.4) (layer "F.Cu") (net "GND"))
 (via (at 155 100.4) (size 0.8) (drill 0.4) (layers "F.Cu" "B.Cu") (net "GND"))
 (via (at 154.7 97.9) (size 0.8) (drill 0.4) (layers "F.Cu" "B.Cu") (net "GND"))
 (via (at 154.5 91.4) (size 0.8) (drill 0.4) (layers "F.Cu" "B.Cu") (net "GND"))
 (via (at 157 88.5) (size 0.8) (drill 0.4) (layers "F.Cu" "B.Cu") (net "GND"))
 (via (at 131.8 103.7) (size 0.8) (drill 0.4) (layers "F.Cu" "B.Cu") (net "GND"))
 (via (at 131.7 101.7) (size 0.8) (drill 0.4) (layers "F.Cu" "B.Cu") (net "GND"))
 (segment (start 154.2 102) (end 157 102) (width 0.4) (layer "F.Cu") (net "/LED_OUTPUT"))
 (segment (start 148.4 101.2) (end 153.4 101.2) (width 0.4) (layer "F.Cu") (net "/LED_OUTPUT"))
 (segment (start 153.4 101.2) (end 154.2 102) (width 0.4) (layer "F.Cu") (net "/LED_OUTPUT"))
 (segment (start 146.0816 102.7785) (end 146.8215 102.7785) (width 0.4) (layer "F.Cu") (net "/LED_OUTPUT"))
 (segment (start 146.8215 102.7785) (end 148.4 101.2) (width 0.4) (layer "F.Cu") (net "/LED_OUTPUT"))
 (segment (start 147.014 97.6985) (end 146.0816 97.6985) (width 0.4) (layer "F.Cu") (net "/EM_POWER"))
 (segment (start 149.6625 95.05) (end 149.35 95.05) (width 0.4) (layer "F.Cu") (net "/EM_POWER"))
 (segment (start 149.6625 95.05) (end 147.014 97.6985) (width 0.4) (layer "F.Cu") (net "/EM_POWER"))
 (segment (start 149.6625 95.05) (end 149.6625 93.175) (width 0.4) (layer "F.Cu") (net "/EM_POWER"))
 (segment (start 151.9375 96) (end 157 96) (width 0.4) (layer "F.Cu") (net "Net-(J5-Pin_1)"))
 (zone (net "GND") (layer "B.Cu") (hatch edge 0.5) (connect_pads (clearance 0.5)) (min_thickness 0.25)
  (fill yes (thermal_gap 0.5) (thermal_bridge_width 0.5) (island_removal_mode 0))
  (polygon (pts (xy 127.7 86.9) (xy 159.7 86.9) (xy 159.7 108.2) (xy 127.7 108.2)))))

